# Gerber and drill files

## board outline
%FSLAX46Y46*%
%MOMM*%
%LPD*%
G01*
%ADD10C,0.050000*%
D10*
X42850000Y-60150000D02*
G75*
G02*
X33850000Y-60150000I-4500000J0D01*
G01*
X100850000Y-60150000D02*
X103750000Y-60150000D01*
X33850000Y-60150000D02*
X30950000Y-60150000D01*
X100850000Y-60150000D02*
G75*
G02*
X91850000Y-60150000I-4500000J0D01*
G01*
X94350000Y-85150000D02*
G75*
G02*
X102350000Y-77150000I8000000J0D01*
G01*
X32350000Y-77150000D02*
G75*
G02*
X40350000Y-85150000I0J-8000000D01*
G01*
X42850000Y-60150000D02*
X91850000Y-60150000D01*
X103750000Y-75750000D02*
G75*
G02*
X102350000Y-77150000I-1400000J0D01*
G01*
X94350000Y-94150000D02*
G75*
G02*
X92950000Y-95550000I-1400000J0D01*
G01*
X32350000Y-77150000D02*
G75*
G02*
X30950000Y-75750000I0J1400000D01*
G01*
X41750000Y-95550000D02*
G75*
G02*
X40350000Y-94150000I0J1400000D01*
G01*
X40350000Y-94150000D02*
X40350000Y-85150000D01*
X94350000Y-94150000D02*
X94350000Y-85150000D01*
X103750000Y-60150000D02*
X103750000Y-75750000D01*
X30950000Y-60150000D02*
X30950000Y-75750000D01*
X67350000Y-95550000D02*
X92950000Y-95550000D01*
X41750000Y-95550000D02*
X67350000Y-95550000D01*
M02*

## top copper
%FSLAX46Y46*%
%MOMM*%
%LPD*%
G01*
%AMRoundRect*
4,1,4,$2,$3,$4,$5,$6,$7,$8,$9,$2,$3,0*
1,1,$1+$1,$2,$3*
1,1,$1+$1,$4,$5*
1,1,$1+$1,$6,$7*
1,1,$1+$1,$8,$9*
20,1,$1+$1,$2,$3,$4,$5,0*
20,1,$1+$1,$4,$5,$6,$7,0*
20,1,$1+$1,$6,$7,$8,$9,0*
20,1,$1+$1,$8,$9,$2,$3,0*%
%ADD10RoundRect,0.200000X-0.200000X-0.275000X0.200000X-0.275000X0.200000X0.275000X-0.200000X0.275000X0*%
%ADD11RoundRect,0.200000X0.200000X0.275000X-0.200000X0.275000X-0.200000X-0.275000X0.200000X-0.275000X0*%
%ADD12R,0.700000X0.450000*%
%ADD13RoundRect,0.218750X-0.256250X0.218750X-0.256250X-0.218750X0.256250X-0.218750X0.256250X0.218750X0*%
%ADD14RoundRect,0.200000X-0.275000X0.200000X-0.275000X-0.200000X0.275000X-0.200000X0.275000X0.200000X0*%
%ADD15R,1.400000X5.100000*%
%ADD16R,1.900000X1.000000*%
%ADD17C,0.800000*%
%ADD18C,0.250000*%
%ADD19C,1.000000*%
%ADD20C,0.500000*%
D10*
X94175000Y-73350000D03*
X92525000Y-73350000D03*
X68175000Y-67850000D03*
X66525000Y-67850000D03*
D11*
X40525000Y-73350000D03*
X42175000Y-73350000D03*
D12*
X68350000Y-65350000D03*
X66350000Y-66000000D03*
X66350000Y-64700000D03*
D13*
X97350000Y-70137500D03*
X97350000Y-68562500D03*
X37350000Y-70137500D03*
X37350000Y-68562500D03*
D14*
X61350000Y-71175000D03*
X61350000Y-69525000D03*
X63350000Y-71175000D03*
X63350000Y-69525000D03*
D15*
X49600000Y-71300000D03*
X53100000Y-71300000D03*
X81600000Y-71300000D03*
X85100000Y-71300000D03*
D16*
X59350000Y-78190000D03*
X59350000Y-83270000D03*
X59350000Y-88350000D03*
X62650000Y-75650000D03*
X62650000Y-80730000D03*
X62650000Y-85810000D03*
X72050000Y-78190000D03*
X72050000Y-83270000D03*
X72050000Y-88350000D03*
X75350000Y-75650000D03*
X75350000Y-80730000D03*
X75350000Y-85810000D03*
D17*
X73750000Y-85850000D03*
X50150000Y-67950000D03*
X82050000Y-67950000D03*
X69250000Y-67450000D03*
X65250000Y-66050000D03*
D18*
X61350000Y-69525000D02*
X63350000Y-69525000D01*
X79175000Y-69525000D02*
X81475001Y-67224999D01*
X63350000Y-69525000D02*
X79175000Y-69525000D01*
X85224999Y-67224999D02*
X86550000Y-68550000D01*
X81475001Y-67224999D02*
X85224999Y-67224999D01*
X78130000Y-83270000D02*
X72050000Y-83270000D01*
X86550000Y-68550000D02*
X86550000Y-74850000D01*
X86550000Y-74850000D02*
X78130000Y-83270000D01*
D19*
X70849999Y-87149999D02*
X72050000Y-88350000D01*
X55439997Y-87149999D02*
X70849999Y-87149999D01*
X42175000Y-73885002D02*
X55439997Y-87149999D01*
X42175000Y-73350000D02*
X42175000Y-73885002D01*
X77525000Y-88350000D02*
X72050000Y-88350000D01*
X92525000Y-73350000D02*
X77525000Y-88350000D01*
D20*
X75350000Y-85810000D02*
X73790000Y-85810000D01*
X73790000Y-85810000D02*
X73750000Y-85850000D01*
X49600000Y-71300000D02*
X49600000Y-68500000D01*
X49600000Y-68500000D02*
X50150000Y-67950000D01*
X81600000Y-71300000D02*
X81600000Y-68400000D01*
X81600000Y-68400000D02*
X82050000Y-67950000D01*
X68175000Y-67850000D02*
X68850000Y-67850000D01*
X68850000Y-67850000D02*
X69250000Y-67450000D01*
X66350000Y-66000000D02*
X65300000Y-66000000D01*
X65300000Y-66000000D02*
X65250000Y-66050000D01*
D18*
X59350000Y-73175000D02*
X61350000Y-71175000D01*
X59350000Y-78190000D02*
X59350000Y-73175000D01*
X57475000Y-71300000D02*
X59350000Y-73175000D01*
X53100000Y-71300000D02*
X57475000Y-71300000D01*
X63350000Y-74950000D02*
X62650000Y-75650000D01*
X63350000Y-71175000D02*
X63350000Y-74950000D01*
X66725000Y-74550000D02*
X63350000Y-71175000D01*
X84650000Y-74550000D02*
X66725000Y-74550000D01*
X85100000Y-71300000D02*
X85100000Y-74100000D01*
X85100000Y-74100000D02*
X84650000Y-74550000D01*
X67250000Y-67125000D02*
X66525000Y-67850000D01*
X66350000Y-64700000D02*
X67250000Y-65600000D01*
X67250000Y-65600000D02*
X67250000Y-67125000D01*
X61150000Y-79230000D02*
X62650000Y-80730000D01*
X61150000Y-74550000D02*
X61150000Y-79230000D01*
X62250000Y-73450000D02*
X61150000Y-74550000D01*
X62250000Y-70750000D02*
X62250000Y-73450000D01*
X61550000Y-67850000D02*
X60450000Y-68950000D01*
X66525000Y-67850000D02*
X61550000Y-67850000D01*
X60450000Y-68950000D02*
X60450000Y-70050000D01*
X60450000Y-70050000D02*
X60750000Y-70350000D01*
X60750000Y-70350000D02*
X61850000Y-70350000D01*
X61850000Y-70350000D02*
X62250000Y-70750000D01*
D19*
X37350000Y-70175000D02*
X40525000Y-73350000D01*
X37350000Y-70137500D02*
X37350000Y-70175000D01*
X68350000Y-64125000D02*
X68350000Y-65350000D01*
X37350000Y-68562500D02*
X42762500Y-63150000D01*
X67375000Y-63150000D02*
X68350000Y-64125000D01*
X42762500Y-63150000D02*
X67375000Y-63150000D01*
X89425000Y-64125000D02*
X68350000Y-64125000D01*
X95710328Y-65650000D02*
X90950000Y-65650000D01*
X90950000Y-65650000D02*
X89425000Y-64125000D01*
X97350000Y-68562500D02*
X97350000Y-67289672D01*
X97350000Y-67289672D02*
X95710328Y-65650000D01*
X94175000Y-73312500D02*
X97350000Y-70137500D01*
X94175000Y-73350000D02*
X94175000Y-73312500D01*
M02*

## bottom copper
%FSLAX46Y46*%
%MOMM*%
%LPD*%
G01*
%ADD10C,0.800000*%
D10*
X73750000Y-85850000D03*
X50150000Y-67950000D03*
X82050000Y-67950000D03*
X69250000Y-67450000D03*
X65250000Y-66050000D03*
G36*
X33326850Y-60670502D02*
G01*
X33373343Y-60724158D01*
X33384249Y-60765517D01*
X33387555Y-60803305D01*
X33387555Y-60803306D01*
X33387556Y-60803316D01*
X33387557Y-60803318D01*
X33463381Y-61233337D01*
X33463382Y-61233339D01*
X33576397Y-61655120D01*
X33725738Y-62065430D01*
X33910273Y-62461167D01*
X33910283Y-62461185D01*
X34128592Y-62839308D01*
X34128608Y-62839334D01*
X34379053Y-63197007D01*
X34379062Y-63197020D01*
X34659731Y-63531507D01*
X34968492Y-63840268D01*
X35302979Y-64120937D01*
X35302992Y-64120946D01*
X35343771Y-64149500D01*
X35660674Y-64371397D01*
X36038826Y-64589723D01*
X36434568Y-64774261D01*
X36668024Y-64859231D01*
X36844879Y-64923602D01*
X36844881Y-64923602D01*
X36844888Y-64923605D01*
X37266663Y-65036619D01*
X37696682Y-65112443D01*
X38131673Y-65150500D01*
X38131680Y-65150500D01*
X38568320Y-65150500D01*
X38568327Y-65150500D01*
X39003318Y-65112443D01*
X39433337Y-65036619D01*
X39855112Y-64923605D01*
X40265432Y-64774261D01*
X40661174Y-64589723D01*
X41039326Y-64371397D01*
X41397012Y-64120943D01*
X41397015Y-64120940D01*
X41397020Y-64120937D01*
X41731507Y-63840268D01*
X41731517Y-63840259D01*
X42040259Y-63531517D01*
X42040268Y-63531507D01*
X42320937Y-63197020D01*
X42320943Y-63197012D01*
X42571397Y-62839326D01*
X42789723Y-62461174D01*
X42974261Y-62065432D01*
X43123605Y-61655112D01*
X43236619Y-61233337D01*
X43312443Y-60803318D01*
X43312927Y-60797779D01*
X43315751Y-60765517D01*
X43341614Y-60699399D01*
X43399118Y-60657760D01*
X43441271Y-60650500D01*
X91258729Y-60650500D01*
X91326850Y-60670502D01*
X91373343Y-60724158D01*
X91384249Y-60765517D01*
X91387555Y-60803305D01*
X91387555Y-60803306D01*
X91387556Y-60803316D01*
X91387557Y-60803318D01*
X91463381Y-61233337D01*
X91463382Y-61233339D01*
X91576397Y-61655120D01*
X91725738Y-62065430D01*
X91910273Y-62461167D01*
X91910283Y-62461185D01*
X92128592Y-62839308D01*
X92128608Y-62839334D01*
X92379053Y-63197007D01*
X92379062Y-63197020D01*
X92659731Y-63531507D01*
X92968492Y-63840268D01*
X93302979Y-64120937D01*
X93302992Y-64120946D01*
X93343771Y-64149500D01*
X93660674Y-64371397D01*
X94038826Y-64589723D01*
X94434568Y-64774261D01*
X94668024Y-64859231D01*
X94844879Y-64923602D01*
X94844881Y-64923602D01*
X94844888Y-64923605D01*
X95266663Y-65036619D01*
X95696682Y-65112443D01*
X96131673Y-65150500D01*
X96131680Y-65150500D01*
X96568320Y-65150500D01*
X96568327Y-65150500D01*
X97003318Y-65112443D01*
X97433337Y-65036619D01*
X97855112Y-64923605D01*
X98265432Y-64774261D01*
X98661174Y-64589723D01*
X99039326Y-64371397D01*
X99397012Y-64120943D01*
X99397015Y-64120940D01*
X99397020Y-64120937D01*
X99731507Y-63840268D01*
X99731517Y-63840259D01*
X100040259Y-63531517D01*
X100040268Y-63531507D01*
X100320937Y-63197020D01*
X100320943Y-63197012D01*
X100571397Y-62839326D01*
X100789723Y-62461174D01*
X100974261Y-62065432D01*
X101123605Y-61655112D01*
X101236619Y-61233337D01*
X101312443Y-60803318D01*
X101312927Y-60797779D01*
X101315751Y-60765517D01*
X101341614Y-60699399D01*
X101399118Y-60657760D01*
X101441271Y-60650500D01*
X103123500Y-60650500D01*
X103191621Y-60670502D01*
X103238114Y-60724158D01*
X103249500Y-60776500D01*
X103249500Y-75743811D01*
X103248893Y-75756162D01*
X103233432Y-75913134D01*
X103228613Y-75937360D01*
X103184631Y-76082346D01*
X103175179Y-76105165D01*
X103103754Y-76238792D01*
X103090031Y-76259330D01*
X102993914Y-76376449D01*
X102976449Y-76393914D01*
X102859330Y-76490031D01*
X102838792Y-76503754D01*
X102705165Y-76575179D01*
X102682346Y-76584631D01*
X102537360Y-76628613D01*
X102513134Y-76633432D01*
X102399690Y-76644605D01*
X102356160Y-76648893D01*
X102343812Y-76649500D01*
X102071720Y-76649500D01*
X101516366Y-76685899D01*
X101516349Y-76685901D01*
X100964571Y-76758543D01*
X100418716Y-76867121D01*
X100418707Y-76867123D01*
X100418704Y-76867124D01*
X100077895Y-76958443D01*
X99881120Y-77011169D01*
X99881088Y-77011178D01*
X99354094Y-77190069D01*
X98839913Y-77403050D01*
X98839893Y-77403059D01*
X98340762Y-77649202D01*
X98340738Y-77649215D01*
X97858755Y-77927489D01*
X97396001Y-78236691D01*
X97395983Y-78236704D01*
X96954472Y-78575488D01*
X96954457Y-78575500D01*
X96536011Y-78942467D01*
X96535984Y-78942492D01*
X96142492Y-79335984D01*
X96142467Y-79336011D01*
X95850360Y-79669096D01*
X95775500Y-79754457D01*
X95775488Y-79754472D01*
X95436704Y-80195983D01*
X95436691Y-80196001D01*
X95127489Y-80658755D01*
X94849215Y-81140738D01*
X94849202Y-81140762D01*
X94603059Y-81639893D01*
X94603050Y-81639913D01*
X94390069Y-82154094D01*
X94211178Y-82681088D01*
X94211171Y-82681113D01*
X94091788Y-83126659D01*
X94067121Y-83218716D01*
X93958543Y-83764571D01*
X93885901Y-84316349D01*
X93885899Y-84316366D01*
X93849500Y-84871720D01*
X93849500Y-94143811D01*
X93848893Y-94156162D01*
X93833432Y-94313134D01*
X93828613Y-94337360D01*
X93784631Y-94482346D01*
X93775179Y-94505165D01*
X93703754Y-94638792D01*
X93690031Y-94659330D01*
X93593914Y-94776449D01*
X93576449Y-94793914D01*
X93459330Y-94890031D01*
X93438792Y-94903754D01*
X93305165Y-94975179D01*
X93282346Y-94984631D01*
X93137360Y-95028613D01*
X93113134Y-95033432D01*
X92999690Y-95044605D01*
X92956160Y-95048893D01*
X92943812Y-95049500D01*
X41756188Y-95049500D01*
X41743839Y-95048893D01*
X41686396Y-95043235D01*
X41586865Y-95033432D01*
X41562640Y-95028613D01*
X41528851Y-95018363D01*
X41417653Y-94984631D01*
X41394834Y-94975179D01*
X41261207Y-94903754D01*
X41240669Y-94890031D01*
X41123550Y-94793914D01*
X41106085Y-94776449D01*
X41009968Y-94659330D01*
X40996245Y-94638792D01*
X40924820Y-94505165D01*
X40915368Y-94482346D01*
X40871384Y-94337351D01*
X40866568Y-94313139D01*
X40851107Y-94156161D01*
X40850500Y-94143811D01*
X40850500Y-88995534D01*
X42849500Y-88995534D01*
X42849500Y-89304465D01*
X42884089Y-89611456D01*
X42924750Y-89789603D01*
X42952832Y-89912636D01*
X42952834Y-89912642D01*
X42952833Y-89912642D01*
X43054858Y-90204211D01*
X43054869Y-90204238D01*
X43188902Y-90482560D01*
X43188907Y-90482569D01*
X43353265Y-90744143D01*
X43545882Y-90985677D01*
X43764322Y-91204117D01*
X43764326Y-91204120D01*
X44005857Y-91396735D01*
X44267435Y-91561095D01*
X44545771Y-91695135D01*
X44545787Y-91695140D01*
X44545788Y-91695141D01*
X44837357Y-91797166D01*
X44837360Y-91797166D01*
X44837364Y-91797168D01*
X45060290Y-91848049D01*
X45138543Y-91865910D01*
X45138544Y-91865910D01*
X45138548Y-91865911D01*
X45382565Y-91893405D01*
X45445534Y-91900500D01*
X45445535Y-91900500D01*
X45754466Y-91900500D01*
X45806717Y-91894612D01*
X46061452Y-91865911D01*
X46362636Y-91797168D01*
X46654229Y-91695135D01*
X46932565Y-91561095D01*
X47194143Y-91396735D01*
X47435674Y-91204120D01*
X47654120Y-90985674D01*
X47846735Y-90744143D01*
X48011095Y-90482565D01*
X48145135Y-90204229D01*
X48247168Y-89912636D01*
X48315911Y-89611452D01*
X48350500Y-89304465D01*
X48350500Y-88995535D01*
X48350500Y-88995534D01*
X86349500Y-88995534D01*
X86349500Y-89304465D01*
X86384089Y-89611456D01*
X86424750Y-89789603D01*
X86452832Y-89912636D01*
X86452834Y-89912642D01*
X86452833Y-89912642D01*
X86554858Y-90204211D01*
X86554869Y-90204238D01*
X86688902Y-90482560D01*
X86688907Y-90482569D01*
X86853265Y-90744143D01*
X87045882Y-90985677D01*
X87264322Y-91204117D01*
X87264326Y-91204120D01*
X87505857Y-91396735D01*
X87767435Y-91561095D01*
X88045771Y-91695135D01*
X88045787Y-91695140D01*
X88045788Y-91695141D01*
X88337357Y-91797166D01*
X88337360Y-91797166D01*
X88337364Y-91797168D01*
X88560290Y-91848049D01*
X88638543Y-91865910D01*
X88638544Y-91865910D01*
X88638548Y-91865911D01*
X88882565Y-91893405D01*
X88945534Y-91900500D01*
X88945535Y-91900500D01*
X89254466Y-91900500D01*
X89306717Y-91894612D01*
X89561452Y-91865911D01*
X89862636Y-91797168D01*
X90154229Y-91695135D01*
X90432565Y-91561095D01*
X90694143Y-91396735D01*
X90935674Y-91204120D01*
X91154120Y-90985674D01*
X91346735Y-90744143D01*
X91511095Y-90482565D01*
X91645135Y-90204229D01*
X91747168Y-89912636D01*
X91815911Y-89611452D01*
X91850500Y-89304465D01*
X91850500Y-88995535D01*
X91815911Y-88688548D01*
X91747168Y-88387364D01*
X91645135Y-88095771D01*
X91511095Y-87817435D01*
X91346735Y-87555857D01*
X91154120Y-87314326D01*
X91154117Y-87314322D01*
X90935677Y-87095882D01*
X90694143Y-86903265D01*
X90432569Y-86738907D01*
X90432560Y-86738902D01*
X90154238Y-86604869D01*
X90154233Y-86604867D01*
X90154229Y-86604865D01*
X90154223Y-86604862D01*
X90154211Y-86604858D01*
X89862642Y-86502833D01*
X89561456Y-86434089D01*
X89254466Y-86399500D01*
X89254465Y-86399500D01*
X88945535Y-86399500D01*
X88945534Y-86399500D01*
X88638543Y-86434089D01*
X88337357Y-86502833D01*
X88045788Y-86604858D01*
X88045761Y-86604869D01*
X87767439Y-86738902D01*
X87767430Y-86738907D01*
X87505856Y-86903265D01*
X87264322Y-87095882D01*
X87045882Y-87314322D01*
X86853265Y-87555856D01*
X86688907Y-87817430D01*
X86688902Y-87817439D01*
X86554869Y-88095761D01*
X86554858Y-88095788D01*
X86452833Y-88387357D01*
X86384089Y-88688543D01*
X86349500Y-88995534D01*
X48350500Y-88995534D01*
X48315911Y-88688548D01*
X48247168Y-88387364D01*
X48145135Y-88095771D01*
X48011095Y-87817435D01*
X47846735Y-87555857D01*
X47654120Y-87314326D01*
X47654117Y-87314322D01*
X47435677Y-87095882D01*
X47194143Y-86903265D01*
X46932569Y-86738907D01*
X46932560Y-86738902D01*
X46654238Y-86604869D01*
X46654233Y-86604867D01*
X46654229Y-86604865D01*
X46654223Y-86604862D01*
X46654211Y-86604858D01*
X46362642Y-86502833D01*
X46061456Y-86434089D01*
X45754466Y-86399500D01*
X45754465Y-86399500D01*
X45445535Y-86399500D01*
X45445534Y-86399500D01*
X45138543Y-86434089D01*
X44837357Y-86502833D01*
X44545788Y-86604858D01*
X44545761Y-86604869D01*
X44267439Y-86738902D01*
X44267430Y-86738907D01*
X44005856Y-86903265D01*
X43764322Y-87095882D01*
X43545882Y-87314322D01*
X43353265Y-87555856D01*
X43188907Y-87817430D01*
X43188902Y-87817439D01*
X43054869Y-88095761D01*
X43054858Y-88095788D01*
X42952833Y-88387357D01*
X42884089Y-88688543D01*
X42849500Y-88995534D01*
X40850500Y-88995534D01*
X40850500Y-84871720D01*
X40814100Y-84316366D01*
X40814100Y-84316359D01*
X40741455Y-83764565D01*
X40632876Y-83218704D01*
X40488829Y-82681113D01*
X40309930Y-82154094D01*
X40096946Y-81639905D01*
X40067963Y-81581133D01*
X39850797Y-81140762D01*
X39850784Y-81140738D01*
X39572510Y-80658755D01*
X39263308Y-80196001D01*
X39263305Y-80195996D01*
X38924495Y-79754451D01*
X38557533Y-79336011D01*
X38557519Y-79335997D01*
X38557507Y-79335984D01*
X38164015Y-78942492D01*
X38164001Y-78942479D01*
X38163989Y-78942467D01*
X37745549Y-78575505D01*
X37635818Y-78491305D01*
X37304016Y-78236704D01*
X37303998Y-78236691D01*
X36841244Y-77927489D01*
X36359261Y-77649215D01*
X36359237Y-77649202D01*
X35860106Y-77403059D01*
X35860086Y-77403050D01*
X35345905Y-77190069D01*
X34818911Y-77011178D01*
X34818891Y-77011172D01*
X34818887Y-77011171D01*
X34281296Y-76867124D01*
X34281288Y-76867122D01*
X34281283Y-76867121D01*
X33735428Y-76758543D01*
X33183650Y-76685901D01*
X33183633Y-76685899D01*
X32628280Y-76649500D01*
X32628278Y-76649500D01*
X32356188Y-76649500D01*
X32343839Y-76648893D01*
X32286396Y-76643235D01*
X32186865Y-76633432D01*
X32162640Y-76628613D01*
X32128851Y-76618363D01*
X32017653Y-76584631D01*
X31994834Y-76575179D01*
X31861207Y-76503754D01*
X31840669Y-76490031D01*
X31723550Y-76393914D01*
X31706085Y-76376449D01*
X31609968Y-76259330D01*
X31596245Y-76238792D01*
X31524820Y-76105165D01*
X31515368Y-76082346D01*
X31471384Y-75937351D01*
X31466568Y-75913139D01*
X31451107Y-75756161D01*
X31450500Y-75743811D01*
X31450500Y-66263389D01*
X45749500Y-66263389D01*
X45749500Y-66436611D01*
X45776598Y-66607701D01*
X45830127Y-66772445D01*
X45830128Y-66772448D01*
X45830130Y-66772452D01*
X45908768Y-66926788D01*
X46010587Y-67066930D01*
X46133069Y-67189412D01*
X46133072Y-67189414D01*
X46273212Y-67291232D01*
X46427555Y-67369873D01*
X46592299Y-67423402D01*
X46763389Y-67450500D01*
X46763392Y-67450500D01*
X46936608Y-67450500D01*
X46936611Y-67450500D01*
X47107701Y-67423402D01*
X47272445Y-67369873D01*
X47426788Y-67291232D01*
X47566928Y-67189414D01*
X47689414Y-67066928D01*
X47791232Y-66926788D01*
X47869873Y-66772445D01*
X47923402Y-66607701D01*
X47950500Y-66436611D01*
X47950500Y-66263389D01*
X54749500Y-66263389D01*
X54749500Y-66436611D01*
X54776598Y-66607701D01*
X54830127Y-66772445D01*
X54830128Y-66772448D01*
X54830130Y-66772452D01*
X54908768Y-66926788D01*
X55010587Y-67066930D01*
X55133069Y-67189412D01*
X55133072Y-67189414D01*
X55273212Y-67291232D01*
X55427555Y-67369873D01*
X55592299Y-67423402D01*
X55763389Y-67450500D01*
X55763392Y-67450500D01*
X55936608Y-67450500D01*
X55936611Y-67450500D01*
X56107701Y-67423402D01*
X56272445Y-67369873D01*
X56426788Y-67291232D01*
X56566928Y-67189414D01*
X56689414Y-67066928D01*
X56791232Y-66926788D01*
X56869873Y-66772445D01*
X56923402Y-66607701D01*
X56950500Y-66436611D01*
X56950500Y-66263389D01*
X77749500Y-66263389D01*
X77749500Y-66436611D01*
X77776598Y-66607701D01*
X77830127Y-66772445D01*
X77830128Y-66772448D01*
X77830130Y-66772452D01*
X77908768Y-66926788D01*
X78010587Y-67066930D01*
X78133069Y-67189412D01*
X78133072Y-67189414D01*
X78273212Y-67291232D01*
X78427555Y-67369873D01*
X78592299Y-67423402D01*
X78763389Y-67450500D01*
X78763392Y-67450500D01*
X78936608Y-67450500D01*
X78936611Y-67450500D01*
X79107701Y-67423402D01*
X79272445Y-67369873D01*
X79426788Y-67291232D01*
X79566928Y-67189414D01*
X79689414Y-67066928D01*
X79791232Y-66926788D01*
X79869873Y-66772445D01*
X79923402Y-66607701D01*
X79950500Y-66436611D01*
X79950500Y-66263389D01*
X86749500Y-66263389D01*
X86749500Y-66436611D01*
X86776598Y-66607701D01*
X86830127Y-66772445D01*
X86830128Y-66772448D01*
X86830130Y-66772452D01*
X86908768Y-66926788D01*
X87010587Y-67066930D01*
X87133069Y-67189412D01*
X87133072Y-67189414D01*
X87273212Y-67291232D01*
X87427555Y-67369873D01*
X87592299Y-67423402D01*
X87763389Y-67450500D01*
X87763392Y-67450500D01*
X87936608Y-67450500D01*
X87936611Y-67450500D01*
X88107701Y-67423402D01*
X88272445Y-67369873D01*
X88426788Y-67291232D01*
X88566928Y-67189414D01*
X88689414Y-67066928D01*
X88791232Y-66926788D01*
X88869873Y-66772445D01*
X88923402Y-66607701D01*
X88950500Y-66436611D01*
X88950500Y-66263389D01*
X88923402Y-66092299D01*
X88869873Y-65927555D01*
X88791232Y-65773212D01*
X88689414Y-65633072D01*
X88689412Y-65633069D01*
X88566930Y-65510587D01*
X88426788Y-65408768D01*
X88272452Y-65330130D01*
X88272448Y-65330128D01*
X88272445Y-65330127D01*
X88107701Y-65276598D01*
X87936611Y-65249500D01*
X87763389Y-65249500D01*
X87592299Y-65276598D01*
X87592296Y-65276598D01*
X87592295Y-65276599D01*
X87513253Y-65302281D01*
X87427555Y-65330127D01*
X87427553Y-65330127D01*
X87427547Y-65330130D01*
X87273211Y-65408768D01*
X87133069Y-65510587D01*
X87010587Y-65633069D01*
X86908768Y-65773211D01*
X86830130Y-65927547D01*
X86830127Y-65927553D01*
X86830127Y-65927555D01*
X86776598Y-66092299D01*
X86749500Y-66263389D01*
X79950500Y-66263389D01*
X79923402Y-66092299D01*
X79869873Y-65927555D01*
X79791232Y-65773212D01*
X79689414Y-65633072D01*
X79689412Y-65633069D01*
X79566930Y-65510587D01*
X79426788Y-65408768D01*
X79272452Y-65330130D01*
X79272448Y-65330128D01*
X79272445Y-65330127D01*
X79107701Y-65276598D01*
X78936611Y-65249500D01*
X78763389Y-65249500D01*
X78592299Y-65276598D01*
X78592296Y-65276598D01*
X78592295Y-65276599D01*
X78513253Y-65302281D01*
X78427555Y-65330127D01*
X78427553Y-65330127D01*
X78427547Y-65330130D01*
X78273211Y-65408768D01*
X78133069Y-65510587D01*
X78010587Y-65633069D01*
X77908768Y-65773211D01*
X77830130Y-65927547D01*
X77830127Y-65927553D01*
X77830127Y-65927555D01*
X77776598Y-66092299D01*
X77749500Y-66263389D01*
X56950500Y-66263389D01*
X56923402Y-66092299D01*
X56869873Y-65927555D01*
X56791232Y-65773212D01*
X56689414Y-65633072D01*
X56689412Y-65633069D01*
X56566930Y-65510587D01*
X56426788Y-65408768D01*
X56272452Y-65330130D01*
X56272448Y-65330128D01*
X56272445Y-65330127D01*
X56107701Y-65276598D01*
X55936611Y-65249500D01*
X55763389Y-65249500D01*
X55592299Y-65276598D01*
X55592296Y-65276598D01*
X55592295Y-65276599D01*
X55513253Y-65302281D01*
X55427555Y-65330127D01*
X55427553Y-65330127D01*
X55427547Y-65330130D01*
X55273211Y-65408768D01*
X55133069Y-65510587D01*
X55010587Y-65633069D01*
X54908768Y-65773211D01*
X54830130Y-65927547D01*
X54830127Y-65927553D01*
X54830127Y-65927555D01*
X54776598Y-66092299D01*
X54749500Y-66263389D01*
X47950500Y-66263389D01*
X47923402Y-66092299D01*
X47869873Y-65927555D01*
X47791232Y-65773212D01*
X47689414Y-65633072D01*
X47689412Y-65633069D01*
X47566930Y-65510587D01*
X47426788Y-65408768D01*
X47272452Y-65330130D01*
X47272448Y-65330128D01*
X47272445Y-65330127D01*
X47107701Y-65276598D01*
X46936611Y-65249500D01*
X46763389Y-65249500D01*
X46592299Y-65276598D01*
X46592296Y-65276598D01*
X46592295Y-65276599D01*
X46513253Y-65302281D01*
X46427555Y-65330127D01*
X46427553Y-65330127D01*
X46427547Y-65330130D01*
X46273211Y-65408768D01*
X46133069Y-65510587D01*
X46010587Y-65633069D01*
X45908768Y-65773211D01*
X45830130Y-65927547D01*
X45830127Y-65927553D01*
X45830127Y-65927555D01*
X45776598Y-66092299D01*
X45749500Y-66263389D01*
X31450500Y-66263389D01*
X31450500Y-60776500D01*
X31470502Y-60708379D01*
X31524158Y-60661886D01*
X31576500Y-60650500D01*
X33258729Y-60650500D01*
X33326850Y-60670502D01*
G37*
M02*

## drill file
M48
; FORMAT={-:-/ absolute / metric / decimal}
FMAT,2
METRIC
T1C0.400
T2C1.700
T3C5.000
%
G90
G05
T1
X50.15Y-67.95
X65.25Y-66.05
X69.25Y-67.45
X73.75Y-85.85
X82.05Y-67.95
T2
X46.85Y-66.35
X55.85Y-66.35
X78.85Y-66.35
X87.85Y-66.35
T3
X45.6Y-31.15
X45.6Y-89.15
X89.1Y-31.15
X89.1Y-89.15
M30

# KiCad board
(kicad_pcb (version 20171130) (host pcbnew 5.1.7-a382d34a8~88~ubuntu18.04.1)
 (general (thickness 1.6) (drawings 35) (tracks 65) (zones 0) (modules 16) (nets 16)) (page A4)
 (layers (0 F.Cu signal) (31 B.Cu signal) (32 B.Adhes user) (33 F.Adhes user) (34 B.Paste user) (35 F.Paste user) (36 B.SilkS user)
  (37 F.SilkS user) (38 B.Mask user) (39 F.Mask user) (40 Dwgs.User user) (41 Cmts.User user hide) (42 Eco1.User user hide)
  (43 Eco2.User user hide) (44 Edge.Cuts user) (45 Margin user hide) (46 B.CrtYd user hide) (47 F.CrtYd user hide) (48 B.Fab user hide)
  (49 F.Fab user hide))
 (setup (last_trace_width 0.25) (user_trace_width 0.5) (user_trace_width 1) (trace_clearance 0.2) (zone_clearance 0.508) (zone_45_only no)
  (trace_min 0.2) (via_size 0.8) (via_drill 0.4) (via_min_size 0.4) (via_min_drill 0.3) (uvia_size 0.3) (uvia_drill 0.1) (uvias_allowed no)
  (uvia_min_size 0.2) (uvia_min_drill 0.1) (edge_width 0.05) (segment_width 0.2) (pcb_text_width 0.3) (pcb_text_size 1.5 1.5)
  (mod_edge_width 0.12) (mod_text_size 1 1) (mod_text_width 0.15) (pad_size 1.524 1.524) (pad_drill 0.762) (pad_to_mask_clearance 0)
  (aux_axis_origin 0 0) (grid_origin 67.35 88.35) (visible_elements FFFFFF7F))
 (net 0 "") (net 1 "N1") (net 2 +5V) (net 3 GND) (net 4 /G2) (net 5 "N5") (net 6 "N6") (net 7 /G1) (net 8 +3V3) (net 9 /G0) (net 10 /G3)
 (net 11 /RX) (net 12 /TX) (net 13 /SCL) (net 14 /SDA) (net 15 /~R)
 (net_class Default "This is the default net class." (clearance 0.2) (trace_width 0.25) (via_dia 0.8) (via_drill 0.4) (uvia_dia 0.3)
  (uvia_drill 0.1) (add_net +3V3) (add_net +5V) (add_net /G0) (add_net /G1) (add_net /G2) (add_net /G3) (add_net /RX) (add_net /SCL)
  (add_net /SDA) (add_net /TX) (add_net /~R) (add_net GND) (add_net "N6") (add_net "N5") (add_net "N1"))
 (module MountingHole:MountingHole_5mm (layer F.Cu) (at 89.1 89.15)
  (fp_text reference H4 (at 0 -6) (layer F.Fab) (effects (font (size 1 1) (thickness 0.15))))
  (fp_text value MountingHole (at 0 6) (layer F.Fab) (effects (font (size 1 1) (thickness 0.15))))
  (pad 1 np_thru_hole circle (at 0 0) (size 5 5) (drill 5) (layers *.Cu *.Mask)))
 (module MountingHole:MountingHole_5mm (layer F.Cu) (at 89.1 31.15)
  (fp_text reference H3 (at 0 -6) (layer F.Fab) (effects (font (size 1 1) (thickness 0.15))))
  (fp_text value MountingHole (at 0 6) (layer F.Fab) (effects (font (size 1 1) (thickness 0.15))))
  (pad 1 np_thru_hole circle (at 0 0) (size 5 5) (drill 5) (layers *.Cu *.Mask)))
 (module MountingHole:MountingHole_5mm (layer F.Cu) (at 45.6 89.15)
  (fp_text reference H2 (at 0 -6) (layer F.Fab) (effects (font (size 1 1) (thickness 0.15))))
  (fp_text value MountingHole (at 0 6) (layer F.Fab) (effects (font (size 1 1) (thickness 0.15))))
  (pad 1 np_thru_hole circle (at 0 0) (size 5 5) (drill 5) (layers *.Cu *.Mask)))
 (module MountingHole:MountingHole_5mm (layer F.Cu) (at 45.6 31.15)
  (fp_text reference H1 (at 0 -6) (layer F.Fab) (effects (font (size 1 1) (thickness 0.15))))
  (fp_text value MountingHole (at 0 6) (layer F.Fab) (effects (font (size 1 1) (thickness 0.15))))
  (pad 1 np_thru_hole circle (at 0 0) (size 5 5) (drill 5) (layers *.Cu *.Mask)))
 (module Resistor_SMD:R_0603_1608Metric (layer F.Cu) (at 93.35 73.35)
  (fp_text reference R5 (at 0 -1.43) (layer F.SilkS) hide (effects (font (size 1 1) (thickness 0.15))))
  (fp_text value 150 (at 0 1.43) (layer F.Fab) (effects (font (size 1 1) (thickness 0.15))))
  (pad 2 smd roundrect (at 0.825 0) (size 0.8 0.95) (layers F.Cu F.Paste F.Mask) (roundrect_rratio 0.25) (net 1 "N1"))
  (pad 1 smd roundrect (at -0.825 0) (size 0.8 0.95) (layers F.Cu F.Paste F.Mask) (roundrect_rratio 0.25) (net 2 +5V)))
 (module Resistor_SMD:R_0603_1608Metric (layer F.Cu) (at 67.35 67.85)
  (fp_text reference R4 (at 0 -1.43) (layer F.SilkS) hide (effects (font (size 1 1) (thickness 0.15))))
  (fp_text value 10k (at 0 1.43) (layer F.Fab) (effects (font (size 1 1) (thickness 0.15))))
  (pad 2 smd roundrect (at 0.825 0) (size 0.8 0.95) (layers F.Cu F.Paste F.Mask) (roundrect_rratio 0.25) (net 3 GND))
  (pad 1 smd roundrect (at -0.825 0) (size 0.8 0.95) (layers F.Cu F.Paste F.Mask) (roundrect_rratio 0.25) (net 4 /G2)))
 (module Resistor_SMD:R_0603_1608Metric (layer F.Cu) (at 41.35 73.35 180)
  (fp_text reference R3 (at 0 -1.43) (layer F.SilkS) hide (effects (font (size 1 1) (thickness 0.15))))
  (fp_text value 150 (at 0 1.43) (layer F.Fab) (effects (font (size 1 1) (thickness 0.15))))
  (pad 2 smd roundrect (at 0.825 0 180) (size 0.8 0.95) (layers F.Cu F.Paste F.Mask) (roundrect_rratio 0.25) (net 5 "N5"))
  (pad 1 smd roundrect (at -0.825 0 180) (size 0.8 0.95) (layers F.Cu F.Paste F.Mask) (roundrect_rratio 0.25) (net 2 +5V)))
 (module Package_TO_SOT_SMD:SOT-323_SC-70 (layer F.Cu) (at 67.35 65.35)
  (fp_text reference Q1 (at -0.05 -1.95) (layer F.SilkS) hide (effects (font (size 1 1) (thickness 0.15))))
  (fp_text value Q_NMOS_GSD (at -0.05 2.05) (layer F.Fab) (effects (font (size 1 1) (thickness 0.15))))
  (pad 3 smd rect (at 1 0 270) (size 0.45 0.7) (layers F.Cu F.Paste F.Mask) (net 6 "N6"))
  (pad 2 smd rect (at -1 0.65 270) (size 0.45 0.7) (layers F.Cu F.Paste F.Mask) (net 3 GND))
  (pad 1 smd rect (at -1 -0.65 270) (size 0.45 0.7) (layers F.Cu F.Paste F.Mask) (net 4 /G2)))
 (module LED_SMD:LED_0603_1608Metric (layer F.Cu) (at 97.35 69.35 270)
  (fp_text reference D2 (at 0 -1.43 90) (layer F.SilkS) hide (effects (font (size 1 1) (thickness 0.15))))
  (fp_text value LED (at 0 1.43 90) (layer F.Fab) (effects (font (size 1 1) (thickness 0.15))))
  (pad 2 smd roundrect (at 0.7875 0 270) (size 0.875 0.95) (layers F.Cu F.Paste F.Mask) (roundrect_rratio 0.25) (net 1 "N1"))
  (pad 1 smd roundrect (at -0.7875 0 270) (size 0.875 0.95) (layers F.Cu F.Paste F.Mask) (roundrect_rratio 0.25) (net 6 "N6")))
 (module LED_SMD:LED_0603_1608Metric (layer F.Cu) (at 37.35 69.35 270)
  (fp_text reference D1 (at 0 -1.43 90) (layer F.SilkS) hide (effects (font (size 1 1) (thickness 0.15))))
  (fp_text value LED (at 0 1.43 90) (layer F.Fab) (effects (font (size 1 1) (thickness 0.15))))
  (pad 2 smd roundrect (at 0.7875 0 270) (size 0.875 0.95) (layers F.Cu F.Paste F.Mask) (roundrect_rratio 0.25) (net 5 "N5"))
  (pad 1 smd roundrect (at -0.7875 0 270) (size 0.875 0.95) (layers F.Cu F.Paste F.Mask) (roundrect_rratio 0.25) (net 6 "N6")))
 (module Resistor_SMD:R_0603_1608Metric (layer F.Cu) (at 61.35 70.35 270)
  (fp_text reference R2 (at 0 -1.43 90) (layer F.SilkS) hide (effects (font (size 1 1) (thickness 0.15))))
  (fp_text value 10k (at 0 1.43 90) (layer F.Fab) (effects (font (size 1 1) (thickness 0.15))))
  (pad 2 smd roundrect (at 0.825 0 270) (size 0.8 0.95) (layers F.Cu F.Paste F.Mask) (roundrect_rratio 0.25) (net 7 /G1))
  (pad 1 smd roundrect (at -0.825 0 270) (size 0.8 0.95) (layers F.Cu F.Paste F.Mask) (roundrect_rratio 0.25) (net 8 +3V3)))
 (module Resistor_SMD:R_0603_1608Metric (layer F.Cu) (at 63.35 70.35 270)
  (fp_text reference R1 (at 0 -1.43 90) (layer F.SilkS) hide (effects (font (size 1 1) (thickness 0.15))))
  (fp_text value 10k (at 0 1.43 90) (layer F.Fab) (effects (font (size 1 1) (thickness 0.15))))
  (pad 2 smd roundrect (at 0.825 0 270) (size 0.8 0.95) (layers F.Cu F.Paste F.Mask) (roundrect_rratio 0.25) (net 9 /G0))
  (pad 1 smd roundrect (at -0.825 0 270) (size 0.8 0.95) (layers F.Cu F.Paste F.Mask) (roundrect_rratio 0.25) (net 8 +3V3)))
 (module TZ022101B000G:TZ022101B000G (layer F.Cu) (at 51.35 66.35 180)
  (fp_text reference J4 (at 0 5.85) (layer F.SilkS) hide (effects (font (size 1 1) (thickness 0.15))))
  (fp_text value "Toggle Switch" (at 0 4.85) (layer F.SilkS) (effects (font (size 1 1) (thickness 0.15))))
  (pad 2 smd rect (at 1.75 -4.95 180) (size 1.4 5.1) (layers F.Cu F.Paste F.Mask) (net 3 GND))
  (pad 1 smd rect (at -1.75 -4.95 180) (size 1.4 5.1) (layers F.Cu F.Paste F.Mask) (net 7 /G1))
  (pad "" np_thru_hole circle (at 4.5 0 180) (size 1.7 1.7) (drill 1.7) (layers *.Cu *.Mask))
  (pad "" np_thru_hole circle (at -4.5 0 180) (size 1.7 1.7) (drill 1.7) (layers *.Cu *.Mask)))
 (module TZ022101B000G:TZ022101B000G (layer F.Cu) (at 83.35 66.35 180)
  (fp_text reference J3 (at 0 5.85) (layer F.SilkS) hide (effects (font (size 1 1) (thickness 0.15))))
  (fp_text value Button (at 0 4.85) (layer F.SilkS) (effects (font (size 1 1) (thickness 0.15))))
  (pad 2 smd rect (at 1.75 -4.95 180) (size 1.4 5.1) (layers F.Cu F.Paste F.Mask) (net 3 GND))
  (pad 1 smd rect (at -1.75 -4.95 180) (size 1.4 5.1) (layers F.Cu F.Paste F.Mask) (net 9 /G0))
  (pad "" np_thru_hole circle (at 4.5 0 180) (size 1.7 1.7) (drill 1.7) (layers *.Cu *.Mask))
  (pad "" np_thru_hole circle (at -4.5 0 180) (size 1.7 1.7) (drill 1.7) (layers *.Cu *.Mask)))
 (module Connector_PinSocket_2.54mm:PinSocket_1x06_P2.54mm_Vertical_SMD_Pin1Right (layer F.Cu) (at 61 82 180)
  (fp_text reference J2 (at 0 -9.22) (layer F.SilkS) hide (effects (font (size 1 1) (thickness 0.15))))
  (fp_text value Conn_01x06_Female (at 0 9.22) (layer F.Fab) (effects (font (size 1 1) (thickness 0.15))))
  (pad 5 smd rect (at 1.65 3.81 180) (size 1.9 1) (layers F.Cu F.Paste F.Mask) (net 7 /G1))
  (pad 3 smd rect (at 1.65 -1.27 180) (size 1.9 1) (layers F.Cu F.Paste F.Mask) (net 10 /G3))
  (pad 1 smd rect (at 1.65 -6.35 180) (size 1.9 1) (layers F.Cu F.Paste F.Mask) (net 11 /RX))
  (pad 6 smd rect (at -1.65 6.35 180) (size 1.9 1) (layers F.Cu F.Paste F.Mask) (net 9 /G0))
  (pad 4 smd rect (at -1.65 1.27 180) (size 1.9 1) (layers F.Cu F.Paste F.Mask) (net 4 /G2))
  (pad 2 smd rect (at -1.65 -3.81 180) (size 1.9 1) (layers F.Cu F.Paste F.Mask) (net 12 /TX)))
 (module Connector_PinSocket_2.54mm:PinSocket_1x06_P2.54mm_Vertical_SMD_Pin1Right (layer F.Cu) (at 73.7 82 180)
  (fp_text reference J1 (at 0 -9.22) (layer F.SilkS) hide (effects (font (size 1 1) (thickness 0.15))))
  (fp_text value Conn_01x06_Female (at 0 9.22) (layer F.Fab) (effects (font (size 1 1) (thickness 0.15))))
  (pad 5 smd rect (at 1.65 3.81 180) (size 1.9 1) (layers F.Cu F.Paste F.Mask) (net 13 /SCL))
  (pad 3 smd rect (at 1.65 -1.27 180) (size 1.9 1) (layers F.Cu F.Paste F.Mask) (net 8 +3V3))
  (pad 1 smd rect (at 1.65 -6.35 180) (size 1.9 1) (layers F.Cu F.Paste F.Mask) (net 2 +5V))
  (pad 6 smd rect (at -1.65 6.35 180) (size 1.9 1) (layers F.Cu F.Paste F.Mask) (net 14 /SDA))
  (pad 4 smd rect (at -1.65 1.27 180) (size 1.9 1) (layers F.Cu F.Paste F.Mask) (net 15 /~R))
  (pad 2 smd rect (at -1.65 -3.81 180) (size 1.9 1) (layers F.Cu F.Paste F.Mask) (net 3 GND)))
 (gr_arc (start 38.35 60.15) (end 33.85 60.15) (angle -180) (layer Edge.Cuts) (width 0.05))
 (gr_line (start 100.85 60.15) (end 103.75 60.15) (layer Edge.Cuts) (width 0.05))
 (gr_line (start 33.85 60.15) (end 30.95 60.15) (layer Edge.Cuts) (width 0.05))
 (gr_arc (start 96.35 60.15) (end 91.85 60.15) (angle -180) (layer Edge.Cuts) (width 0.05))
 (gr_arc (start 102.35 85.15) (end 102.35 77.15) (angle -90) (layer Edge.Cuts) (width 0.05))
 (gr_arc (start 32.35 85.15) (end 40.35 85.15) (angle -90) (layer Edge.Cuts) (width 0.05))
 (gr_line (start 42.85 60.15) (end 91.85 60.15) (layer Edge.Cuts) (width 0.05))
 (gr_arc (start 102.35 75.75) (end 102.35 77.15) (angle -90) (layer Edge.Cuts) (width 0.05))
 (gr_arc (start 92.95 94.15) (end 92.95 95.55) (angle -90) (layer Edge.Cuts) (width 0.05))
 (gr_arc (start 32.35 75.75) (end 30.95 75.75) (angle -90) (layer Edge.Cuts) (width 0.05))
 (gr_arc (start 41.75 94.15) (end 40.35 94.15) (angle -90) (layer Edge.Cuts) (width 0.05))
 (gr_line (start 40.35 94.15) (end 40.35 85.15) (layer Edge.Cuts) (width 0.05))
 (gr_line (start 94.35 94.15) (end 94.35 85.15) (layer Edge.Cuts) (width 0.05))
 (gr_line (start 103.75 60.15) (end 103.75 75.75) (layer Edge.Cuts) (width 0.05))
 (gr_line (start 30.95 60.15) (end 30.95 75.75) (layer Edge.Cuts) (width 0.05))
 (gr_line (start 67.35 95.55) (end 92.95 95.55) (layer Edge.Cuts) (width 0.05))
 (gr_line (start 41.75 95.55) (end 67.35 95.55) (layer Edge.Cuts) (width 0.05))
 (segment (start 61.35 69.525) (end 63.35 69.525) (width 0.25) (layer F.Cu) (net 8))
 (segment (start 79.175 69.525) (end 81.475001 67.224999) (width 0.25) (layer F.Cu) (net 8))
 (segment (start 63.35 69.525) (end 79.175 69.525) (width 0.25) (layer F.Cu) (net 8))
 (segment (start 85.224999 67.224999) (end 86.55 68.55) (width 0.25) (layer F.Cu) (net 8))
 (segment (start 81.475001 67.224999) (end 85.224999 67.224999) (width 0.25) (layer F.Cu) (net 8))
 (segment (start 78.13 83.27) (end 72.05 83.27) (width 0.25) (layer F.Cu) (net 8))
 (segment (start 86.55 68.55) (end 86.55 74.85) (width 0.25) (layer F.Cu) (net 8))
 (segment (start 86.55 74.85) (end 78.13 83.27) (width 0.25) (layer F.Cu) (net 8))
 (segment (start 70.849999 87.149999) (end 72.05 88.35) (width 1) (layer F.Cu) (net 2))
 (segment (start 55.439997 87.149999) (end 70.849999 87.149999) (width 1) (layer F.Cu) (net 2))
 (segment (start 42.175 73.885002) (end 55.439997 87.149999) (width 1) (layer F.Cu) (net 2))
 (segment (start 42.175 73.35) (end 42.175 73.885002) (width 1) (layer F.Cu) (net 2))
 (segment (start 77.525 88.35) (end 72.05 88.35) (width 1) (layer F.Cu) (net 2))
 (segment (start 92.525 73.35) (end 77.525 88.35) (width 1) (layer F.Cu) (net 2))
 (via (at 73.75 85.85) (size 0.8) (drill 0.4) (layers F.Cu B.Cu) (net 3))
 (segment (start 75.35 85.81) (end 73.79 85.81) (width 0.5) (layer F.Cu) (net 3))
 (segment (start 73.79 85.81) (end 73.75 85.85) (width 0.5) (layer F.Cu) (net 3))
 (segment (start 49.6 71.3) (end 49.6 68.5) (width 0.5) (layer F.Cu) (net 3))
 (via (at 50.15 67.95) (size 0.8) (drill 0.4) (layers F.Cu B.Cu) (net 3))
 (segment (start 49.6 68.5) (end 50.15 67.95) (width 0.5) (layer F.Cu) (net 3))
 (via (at 82.05 67.95) (size 0.8) (drill 0.4) (layers F.Cu B.Cu) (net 3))
 (segment (start 81.6 71.3) (end 81.6 68.4) (width 0.5) (layer F.Cu) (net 3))
 (segment (start 81.6 68.4) (end 82.05 67.95) (width 0.5) (layer F.Cu) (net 3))
 (segment (start 68.175 67.85) (end 68.85 67.85) (width 0.5) (layer F.Cu) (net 3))
 (via (at 69.25 67.45) (size 0.8) (drill 0.4) (layers F.Cu B.Cu) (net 3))
 (segment (start 68.85 67.85) (end 69.25 67.45) (width 0.5) (layer F.Cu) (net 3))
 (via (at 65.25 66.05) (size 0.8) (drill 0.4) (layers F.Cu B.Cu) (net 3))
 (segment (start 66.35 66) (end 65.3 66) (width 0.5) (layer F.Cu) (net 3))
 (segment (start 65.3 66) (end 65.25 66.05) (width 0.5) (layer F.Cu) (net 3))
 (segment (start 59.35 73.175) (end 61.35 71.175) (width 0.25) (layer F.Cu) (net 7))
 (segment (start 59.35 78.19) (end 59.35 73.175) (width 0.25) (layer F.Cu) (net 7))
 (segment (start 57.475 71.3) (end 59.35 73.175) (width 0.25) (layer F.Cu) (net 7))
 (segment (start 53.1 71.3) (end 57.475 71.3) (width 0.25) (layer F.Cu) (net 7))
 (segment (start 63.35 74.95) (end 62.65 75.65) (width 0.25) (layer F.Cu) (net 9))
 (segment (start 63.35 71.175) (end 63.35 74.95) (width 0.25) (layer F.Cu) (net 9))
 (segment (start 66.725 74.55) (end 63.35 71.175) (width 0.25) (layer F.Cu) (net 9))
 (segment (start 84.65 74.55) (end 66.725 74.55) (width 0.25) (layer F.Cu) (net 9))
 (segment (start 85.1 71.3) (end 85.1 74.1) (width 0.25) (layer F.Cu) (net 9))
 (segment (start 85.1 74.1) (end 84.65 74.55) (width 0.25) (layer F.Cu) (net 9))
 (segment (start 67.25 67.125) (end 66.525 67.85) (width 0.25) (layer F.Cu) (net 4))
 (segment (start 66.35 64.7) (end 67.25 65.6) (width 0.25) (layer F.Cu) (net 4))
 (segment (start 67.25 65.6) (end 67.25 67.125) (width 0.25) (layer F.Cu) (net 4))
 (segment (start 61.15 79.23) (end 62.65 80.73) (width 0.25) (layer F.Cu) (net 4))
 (segment (start 61.15 74.55) (end 61.15 79.23) (width 0.25) (layer F.Cu) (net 4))
 (segment (start 62.25 73.45) (end 61.15 74.55) (width 0.25) (layer F.Cu) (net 4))
 (segment (start 62.25 70.75) (end 62.25 73.45) (width 0.25) (layer F.Cu) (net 4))
 (segment (start 61.55 67.85) (end 60.45 68.95) (width 0.25) (layer F.Cu) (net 4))
 (segment (start 66.525 67.85) (end 61.55 67.85) (width 0.25) (layer F.Cu) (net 4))
 (segment (start 60.45 68.95) (end 60.45 70.05) (width 0.25) (layer F.Cu) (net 4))
 (segment (start 60.45 70.05) (end 60.75 70.35) (width 0.25) (layer F.Cu) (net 4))
 (segment (start 60.75 70.35) (end 61.85 70.35) (width 0.25) (layer F.Cu) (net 4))
 (segment (start 61.85 70.35) (end 62.25 70.75) (width 0.25) (layer F.Cu) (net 4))
 (segment (start 37.35 70.175) (end 40.525 73.35) (width 1) (layer F.Cu) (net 5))
 (segment (start 37.35 70.1375) (end 37.35 70.175) (width 1) (layer F.Cu) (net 5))
 (segment (start 68.35 64.125) (end 68.35 65.35) (width 1) (layer F.Cu) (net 6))
 (segment (start 37.35 68.5625) (end 42.7625 63.15) (width 1) (layer F.Cu) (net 6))
 (segment (start 67.375 63.15) (end 68.35 64.125) (width 1) (layer F.Cu) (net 6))
 (segment (start 42.7625 63.15) (end 67.375 63.15) (width 1) (layer F.Cu) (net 6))
 (segment (start 89.425 64.125) (end 68.35 64.125) (width 1) (layer F.Cu) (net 6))
 (segment (start 95.710328 65.65) (end 90.95 65.65) (width 1) (layer F.Cu) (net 6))
 (segment (start 90.95 65.65) (end 89.425 64.125) (width 1) (layer F.Cu) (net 6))
 (segment (start 97.35 68.5625) (end 97.35 67.289672) (width 1) (layer F.Cu) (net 6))
 (segment (start 97.35 67.289672) (end 95.710328 65.65) (width 1) (layer F.Cu) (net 6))
 (segment (start 94.175 73.3125) (end 97.35 70.1375) (width 1) (layer F.Cu) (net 1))
 (segment (start 94.175 73.35) (end 94.175 73.3125) (width 1) (layer F.Cu) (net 1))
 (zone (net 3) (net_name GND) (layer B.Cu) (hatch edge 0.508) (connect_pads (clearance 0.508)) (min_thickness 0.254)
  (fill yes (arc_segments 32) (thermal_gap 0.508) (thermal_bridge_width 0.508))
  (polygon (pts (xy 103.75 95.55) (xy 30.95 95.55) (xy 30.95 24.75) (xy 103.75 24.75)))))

